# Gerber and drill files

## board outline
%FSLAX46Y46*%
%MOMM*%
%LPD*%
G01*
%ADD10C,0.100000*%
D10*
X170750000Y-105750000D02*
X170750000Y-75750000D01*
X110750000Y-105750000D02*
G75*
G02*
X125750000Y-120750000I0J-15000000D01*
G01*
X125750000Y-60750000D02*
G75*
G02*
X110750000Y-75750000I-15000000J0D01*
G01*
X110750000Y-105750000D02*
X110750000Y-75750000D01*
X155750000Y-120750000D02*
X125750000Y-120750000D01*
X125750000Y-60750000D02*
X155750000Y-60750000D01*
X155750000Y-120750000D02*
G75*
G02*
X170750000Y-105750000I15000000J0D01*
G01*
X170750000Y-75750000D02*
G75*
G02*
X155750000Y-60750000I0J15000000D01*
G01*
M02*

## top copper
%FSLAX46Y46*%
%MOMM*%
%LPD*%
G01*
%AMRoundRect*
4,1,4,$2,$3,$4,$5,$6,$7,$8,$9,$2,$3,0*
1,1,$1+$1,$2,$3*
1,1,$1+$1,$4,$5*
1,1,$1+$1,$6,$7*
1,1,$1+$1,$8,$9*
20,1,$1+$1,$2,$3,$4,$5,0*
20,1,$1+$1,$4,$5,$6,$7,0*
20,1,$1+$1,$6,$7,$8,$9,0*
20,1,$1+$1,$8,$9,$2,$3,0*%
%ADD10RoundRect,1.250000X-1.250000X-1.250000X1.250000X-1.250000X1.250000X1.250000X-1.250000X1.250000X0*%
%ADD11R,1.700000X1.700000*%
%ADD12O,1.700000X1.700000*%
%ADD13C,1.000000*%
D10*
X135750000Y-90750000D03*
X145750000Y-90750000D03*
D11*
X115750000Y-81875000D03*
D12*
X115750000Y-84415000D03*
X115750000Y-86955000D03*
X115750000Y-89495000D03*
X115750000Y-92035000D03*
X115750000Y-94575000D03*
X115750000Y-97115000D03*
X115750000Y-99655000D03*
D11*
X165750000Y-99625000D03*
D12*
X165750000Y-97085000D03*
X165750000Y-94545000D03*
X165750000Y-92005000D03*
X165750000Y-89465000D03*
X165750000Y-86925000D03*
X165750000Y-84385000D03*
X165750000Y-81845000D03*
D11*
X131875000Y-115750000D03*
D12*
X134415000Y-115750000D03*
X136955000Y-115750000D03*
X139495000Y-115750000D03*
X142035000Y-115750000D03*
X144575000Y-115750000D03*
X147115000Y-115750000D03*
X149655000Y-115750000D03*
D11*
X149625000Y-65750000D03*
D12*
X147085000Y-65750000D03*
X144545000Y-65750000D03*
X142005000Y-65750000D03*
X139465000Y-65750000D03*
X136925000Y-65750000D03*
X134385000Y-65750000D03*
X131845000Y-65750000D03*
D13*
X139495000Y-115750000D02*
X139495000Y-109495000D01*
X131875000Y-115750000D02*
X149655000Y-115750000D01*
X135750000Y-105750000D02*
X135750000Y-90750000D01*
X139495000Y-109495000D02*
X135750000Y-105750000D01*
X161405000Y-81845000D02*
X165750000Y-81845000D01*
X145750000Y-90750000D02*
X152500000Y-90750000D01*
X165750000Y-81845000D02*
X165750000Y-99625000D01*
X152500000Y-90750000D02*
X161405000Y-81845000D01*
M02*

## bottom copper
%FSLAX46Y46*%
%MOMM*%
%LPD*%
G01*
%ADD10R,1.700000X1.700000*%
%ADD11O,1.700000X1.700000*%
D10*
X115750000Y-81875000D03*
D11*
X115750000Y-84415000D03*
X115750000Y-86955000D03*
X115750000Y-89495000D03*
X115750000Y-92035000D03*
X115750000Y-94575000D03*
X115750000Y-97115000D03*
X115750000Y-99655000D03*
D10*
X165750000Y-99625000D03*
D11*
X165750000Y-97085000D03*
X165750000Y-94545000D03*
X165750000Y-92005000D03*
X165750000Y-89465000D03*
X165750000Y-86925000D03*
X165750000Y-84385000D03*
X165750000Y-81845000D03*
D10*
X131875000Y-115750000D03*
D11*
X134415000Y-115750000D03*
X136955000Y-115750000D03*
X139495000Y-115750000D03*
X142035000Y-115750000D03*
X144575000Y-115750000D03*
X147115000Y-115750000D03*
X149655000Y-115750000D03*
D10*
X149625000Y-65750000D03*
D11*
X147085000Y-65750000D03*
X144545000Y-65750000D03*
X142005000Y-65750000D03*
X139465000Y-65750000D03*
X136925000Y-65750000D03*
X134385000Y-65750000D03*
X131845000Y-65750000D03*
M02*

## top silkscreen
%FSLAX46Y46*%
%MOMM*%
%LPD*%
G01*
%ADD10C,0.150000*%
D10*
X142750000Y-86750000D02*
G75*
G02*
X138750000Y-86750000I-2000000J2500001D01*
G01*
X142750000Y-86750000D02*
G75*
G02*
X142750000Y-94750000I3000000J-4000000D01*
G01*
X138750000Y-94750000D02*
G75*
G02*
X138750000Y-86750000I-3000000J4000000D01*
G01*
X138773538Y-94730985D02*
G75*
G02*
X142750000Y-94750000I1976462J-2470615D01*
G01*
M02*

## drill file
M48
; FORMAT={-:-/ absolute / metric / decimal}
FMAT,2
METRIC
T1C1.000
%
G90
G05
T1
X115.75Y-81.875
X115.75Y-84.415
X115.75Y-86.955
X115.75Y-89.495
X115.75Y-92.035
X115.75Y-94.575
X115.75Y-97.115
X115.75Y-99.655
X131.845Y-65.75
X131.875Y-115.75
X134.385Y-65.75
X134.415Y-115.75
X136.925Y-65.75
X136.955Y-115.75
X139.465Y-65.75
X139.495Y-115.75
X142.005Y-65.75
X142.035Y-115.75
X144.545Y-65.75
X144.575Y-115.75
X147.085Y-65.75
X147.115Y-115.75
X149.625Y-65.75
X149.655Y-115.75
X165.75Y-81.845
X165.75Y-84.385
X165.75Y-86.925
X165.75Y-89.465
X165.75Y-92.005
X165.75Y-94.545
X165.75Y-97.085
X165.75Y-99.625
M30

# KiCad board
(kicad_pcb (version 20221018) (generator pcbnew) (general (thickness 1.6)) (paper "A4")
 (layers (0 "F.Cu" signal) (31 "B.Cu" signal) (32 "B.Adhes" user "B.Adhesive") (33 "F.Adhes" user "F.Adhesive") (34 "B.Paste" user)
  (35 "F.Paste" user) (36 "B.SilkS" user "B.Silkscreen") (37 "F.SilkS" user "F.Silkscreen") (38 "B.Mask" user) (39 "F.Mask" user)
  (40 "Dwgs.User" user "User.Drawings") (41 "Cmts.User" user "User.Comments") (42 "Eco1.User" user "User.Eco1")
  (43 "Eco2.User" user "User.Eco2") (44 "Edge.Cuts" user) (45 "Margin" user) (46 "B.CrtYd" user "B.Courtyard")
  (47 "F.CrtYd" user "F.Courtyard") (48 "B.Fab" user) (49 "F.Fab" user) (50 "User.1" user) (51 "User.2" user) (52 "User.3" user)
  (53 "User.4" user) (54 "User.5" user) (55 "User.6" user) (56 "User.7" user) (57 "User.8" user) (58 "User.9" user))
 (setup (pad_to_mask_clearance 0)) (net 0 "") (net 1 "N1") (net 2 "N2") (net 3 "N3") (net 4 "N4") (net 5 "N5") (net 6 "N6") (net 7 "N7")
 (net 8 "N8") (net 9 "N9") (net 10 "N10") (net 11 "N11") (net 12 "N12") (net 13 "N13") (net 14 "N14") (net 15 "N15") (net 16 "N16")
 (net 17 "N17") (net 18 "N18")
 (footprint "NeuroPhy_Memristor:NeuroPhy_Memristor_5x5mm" (layer "F.Cu") (at 140.75 90.75)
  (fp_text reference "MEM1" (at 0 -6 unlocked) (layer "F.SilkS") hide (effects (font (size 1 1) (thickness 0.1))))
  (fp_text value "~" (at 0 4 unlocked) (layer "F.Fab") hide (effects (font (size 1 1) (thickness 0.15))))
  (pad "1" smd roundrect (at -5 0) (size 5 5) (layers "F.Cu" "F.Mask") (roundrect_rratio 0.25) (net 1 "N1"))
  (pad "2" smd roundrect (at 5 0) (size 5 5) (layers "F.Cu" "F.Mask") (roundrect_rratio 0.25) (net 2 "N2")))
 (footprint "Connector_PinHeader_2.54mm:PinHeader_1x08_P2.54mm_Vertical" (layer "B.Cu") (at 115.75 81.875 180)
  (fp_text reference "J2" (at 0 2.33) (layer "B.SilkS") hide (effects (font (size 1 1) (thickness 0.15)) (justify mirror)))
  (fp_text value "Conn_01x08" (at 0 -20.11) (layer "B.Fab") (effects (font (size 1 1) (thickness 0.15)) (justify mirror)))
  (pad "1" thru_hole rect (at 0 0 180) (size 1.7 1.7) (drill 1) (layers "*.Cu" "*.Mask") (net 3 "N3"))
  (pad "2" thru_hole oval (at 0 -2.54 180) (size 1.7 1.7) (drill 1) (layers "*.Cu" "*.Mask") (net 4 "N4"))
  (pad "3" thru_hole oval (at 0 -5.08 180) (size 1.7 1.7) (drill 1) (layers "*.Cu" "*.Mask") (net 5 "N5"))
  (pad "4" thru_hole oval (at 0 -7.62 180) (size 1.7 1.7) (drill 1) (layers "*.Cu" "*.Mask") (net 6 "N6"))
  (pad "5" thru_hole oval (at 0 -10.16 180) (size 1.7 1.7) (drill 1) (layers "*.Cu" "*.Mask") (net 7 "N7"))
  (pad "6" thru_hole oval (at 0 -12.7 180) (size 1.7 1.7) (drill 1) (layers "*.Cu" "*.Mask") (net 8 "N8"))
  (pad "7" thru_hole oval (at 0 -15.24 180) (size 1.7 1.7) (drill 1) (layers "*.Cu" "*.Mask") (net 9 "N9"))
  (pad "8" thru_hole oval (at 0 -17.78 180) (size 1.7 1.7) (drill 1) (layers "*.Cu" "*.Mask") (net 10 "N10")))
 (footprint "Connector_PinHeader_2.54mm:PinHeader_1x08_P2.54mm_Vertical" (layer "B.Cu") (at 165.75 99.625)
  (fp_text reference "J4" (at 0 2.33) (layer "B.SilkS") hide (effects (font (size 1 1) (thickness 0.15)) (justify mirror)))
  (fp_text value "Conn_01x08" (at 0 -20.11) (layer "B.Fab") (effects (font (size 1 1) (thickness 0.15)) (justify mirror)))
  (pad "1" thru_hole rect (at 0 0) (size 1.7 1.7) (drill 1) (layers "*.Cu" "*.Mask") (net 2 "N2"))
  (pad "2" thru_hole oval (at 0 -2.54) (size 1.7 1.7) (drill 1) (layers "*.Cu" "*.Mask") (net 2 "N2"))
  (pad "3" thru_hole oval (at 0 -5.08) (size 1.7 1.7) (drill 1) (layers "*.Cu" "*.Mask") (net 2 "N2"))
  (pad "4" thru_hole oval (at 0 -7.62) (size 1.7 1.7) (drill 1) (layers "*.Cu" "*.Mask") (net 2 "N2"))
  (pad "5" thru_hole oval (at 0 -10.16) (size 1.7 1.7) (drill 1) (layers "*.Cu" "*.Mask") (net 2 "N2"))
  (pad "6" thru_hole oval (at 0 -12.7) (size 1.7 1.7) (drill 1) (layers "*.Cu" "*.Mask") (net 2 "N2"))
  (pad "7" thru_hole oval (at 0 -15.24) (size 1.7 1.7) (drill 1) (layers "*.Cu" "*.Mask") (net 2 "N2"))
  (pad "8" thru_hole oval (at 0 -17.78) (size 1.7 1.7) (drill 1) (layers "*.Cu" "*.Mask") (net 2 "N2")))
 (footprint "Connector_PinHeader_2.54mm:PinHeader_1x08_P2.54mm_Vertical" (layer "B.Cu") (at 131.875 115.75 -90)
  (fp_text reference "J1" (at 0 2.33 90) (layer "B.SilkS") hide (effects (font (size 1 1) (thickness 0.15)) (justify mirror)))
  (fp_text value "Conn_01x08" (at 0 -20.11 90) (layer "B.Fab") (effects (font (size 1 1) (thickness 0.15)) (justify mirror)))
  (pad "1" thru_hole rect (at 0 0 270) (size 1.7 1.7) (drill 1) (layers "*.Cu" "*.Mask") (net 1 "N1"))
  (pad "2" thru_hole oval (at 0 -2.54 270) (size 1.7 1.7) (drill 1) (layers "*.Cu" "*.Mask") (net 1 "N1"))
  (pad "3" thru_hole oval (at 0 -5.08 270) (size 1.7 1.7) (drill 1) (layers "*.Cu" "*.Mask") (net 1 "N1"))
  (pad "4" thru_hole oval (at 0 -7.62 270) (size 1.7 1.7) (drill 1) (layers "*.Cu" "*.Mask") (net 1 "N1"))
  (pad "5" thru_hole oval (at 0 -10.16 270) (size 1.7 1.7) (drill 1) (layers "*.Cu" "*.Mask") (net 1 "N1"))
  (pad "6" thru_hole oval (at 0 -12.7 270) (size 1.7 1.7) (drill 1) (layers "*.Cu" "*.Mask") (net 1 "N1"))
  (pad "7" thru_hole oval (at 0 -15.24 270) (size 1.7 1.7) (drill 1) (layers "*.Cu" "*.Mask") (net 1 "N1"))
  (pad "8" thru_hole oval (at 0 -17.78 270) (size 1.7 1.7) (drill 1) (layers "*.Cu" "*.Mask") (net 1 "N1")))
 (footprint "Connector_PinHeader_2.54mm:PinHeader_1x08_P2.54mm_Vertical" (layer "B.Cu") (at 149.625 65.75 90)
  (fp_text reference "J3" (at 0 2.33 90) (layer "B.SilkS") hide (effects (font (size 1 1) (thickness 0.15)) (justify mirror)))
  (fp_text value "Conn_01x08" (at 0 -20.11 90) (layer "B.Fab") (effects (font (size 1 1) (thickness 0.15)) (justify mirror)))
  (pad "1" thru_hole rect (at 0 0 90) (size 1.7 1.7) (drill 1) (layers "*.Cu" "*.Mask") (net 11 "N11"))
  (pad "2" thru_hole oval (at 0 -2.54 90) (size 1.7 1.7) (drill 1) (layers "*.Cu" "*.Mask") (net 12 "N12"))
  (pad "3" thru_hole oval (at 0 -5.08 90) (size 1.7 1.7) (drill 1) (layers "*.Cu" "*.Mask") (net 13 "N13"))
  (pad "4" thru_hole oval (at 0 -7.62 90) (size 1.7 1.7) (drill 1) (layers "*.Cu" "*.Mask") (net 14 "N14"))
  (pad "5" thru_hole oval (at 0 -10.16 90) (size 1.7 1.7) (drill 1) (layers "*.Cu" "*.Mask") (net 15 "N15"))
  (pad "6" thru_hole oval (at 0 -12.7 90) (size 1.7 1.7) (drill 1) (layers "*.Cu" "*.Mask") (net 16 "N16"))
  (pad "7" thru_hole oval (at 0 -15.24 90) (size 1.7 1.7) (drill 1) (layers "*.Cu" "*.Mask") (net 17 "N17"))
  (pad "8" thru_hole oval (at 0 -17.78 90) (size 1.7 1.7) (drill 1) (layers "*.Cu" "*.Mask") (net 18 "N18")))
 (gr_arc (start 142.75 86.75) (mid 140.75 87.451562) (end 138.75 86.75) (stroke (width 0.15) (type default)) (layer "F.SilkS"))
 (gr_arc (start 142.75 86.75) (mid 150.75 90.75) (end 142.75 94.75) (stroke (width 0.15) (type default)) (layer "F.SilkS"))
 (gr_arc (start 138.75 94.75) (mid 130.75 90.75) (end 138.75 86.75) (stroke (width 0.15) (type default)) (layer "F.SilkS"))
 (gr_arc (start 138.773538 94.730985) (mid 140.765129 94.037716) (end 142.749999 94.750001) (stroke (width 0.15) (type default))
  (layer "F.SilkS"))
 (gr_line (start 170.75 105.75) (end 170.75 75.75) (stroke (width 0.1) (type default)) (layer "Edge.Cuts"))
 (gr_arc (start 110.75 105.75) (mid 121.356602 110.143398) (end 125.75 120.75) (stroke (width 0.1) (type default)) (layer "Edge.Cuts"))
 (gr_arc (start 125.75 60.75) (mid 121.356602 71.356602) (end 110.75 75.75) (stroke (width 0.1) (type default)) (layer "Edge.Cuts"))
 (gr_line (start 110.75 105.75) (end 110.75 75.75) (stroke (width 0.1) (type default)) (layer "Edge.Cuts"))
 (gr_line (start 155.75 120.75) (end 125.75 120.75) (stroke (width 0.1) (type default)) (layer "Edge.Cuts"))
 (gr_line (start 125.75 60.75) (end 155.75 60.75) (stroke (width 0.1) (type default)) (layer "Edge.Cuts"))
 (gr_arc (start 155.75 120.75) (mid 160.143398 110.143398) (end 170.75 105.75) (stroke (width 0.1) (type default)) (layer "Edge.Cuts"))
 (gr_arc (start 170.75 75.75) (mid 160.143398 71.356602) (end 155.75 60.75) (stroke (width 0.1) (type default)) (layer "Edge.Cuts"))
 (segment (start 139.495 115.75) (end 139.495 109.495) (width 1) (layer "F.Cu") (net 1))
 (segment (start 131.875 115.75) (end 149.655 115.75) (width 1) (layer "F.Cu") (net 1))
 (segment (start 135.75 105.75) (end 135.75 90.75) (width 1) (layer "F.Cu") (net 1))
 (segment (start 139.495 109.495) (end 135.75 105.75) (width 1) (layer "F.Cu") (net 1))
 (segment (start 161.405 81.845) (end 165.75 81.845) (width 1) (layer "F.Cu") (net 2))
 (segment (start 145.75 90.75) (end 152.5 90.75) (width 1) (layer "F.Cu") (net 2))
 (segment (start 165.75 81.845) (end 165.75 99.625) (width 1) (layer "F.Cu") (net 2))
 (segment (start 152.5 90.75) (end 161.405 81.845) (width 1) (layer "F.Cu") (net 2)))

